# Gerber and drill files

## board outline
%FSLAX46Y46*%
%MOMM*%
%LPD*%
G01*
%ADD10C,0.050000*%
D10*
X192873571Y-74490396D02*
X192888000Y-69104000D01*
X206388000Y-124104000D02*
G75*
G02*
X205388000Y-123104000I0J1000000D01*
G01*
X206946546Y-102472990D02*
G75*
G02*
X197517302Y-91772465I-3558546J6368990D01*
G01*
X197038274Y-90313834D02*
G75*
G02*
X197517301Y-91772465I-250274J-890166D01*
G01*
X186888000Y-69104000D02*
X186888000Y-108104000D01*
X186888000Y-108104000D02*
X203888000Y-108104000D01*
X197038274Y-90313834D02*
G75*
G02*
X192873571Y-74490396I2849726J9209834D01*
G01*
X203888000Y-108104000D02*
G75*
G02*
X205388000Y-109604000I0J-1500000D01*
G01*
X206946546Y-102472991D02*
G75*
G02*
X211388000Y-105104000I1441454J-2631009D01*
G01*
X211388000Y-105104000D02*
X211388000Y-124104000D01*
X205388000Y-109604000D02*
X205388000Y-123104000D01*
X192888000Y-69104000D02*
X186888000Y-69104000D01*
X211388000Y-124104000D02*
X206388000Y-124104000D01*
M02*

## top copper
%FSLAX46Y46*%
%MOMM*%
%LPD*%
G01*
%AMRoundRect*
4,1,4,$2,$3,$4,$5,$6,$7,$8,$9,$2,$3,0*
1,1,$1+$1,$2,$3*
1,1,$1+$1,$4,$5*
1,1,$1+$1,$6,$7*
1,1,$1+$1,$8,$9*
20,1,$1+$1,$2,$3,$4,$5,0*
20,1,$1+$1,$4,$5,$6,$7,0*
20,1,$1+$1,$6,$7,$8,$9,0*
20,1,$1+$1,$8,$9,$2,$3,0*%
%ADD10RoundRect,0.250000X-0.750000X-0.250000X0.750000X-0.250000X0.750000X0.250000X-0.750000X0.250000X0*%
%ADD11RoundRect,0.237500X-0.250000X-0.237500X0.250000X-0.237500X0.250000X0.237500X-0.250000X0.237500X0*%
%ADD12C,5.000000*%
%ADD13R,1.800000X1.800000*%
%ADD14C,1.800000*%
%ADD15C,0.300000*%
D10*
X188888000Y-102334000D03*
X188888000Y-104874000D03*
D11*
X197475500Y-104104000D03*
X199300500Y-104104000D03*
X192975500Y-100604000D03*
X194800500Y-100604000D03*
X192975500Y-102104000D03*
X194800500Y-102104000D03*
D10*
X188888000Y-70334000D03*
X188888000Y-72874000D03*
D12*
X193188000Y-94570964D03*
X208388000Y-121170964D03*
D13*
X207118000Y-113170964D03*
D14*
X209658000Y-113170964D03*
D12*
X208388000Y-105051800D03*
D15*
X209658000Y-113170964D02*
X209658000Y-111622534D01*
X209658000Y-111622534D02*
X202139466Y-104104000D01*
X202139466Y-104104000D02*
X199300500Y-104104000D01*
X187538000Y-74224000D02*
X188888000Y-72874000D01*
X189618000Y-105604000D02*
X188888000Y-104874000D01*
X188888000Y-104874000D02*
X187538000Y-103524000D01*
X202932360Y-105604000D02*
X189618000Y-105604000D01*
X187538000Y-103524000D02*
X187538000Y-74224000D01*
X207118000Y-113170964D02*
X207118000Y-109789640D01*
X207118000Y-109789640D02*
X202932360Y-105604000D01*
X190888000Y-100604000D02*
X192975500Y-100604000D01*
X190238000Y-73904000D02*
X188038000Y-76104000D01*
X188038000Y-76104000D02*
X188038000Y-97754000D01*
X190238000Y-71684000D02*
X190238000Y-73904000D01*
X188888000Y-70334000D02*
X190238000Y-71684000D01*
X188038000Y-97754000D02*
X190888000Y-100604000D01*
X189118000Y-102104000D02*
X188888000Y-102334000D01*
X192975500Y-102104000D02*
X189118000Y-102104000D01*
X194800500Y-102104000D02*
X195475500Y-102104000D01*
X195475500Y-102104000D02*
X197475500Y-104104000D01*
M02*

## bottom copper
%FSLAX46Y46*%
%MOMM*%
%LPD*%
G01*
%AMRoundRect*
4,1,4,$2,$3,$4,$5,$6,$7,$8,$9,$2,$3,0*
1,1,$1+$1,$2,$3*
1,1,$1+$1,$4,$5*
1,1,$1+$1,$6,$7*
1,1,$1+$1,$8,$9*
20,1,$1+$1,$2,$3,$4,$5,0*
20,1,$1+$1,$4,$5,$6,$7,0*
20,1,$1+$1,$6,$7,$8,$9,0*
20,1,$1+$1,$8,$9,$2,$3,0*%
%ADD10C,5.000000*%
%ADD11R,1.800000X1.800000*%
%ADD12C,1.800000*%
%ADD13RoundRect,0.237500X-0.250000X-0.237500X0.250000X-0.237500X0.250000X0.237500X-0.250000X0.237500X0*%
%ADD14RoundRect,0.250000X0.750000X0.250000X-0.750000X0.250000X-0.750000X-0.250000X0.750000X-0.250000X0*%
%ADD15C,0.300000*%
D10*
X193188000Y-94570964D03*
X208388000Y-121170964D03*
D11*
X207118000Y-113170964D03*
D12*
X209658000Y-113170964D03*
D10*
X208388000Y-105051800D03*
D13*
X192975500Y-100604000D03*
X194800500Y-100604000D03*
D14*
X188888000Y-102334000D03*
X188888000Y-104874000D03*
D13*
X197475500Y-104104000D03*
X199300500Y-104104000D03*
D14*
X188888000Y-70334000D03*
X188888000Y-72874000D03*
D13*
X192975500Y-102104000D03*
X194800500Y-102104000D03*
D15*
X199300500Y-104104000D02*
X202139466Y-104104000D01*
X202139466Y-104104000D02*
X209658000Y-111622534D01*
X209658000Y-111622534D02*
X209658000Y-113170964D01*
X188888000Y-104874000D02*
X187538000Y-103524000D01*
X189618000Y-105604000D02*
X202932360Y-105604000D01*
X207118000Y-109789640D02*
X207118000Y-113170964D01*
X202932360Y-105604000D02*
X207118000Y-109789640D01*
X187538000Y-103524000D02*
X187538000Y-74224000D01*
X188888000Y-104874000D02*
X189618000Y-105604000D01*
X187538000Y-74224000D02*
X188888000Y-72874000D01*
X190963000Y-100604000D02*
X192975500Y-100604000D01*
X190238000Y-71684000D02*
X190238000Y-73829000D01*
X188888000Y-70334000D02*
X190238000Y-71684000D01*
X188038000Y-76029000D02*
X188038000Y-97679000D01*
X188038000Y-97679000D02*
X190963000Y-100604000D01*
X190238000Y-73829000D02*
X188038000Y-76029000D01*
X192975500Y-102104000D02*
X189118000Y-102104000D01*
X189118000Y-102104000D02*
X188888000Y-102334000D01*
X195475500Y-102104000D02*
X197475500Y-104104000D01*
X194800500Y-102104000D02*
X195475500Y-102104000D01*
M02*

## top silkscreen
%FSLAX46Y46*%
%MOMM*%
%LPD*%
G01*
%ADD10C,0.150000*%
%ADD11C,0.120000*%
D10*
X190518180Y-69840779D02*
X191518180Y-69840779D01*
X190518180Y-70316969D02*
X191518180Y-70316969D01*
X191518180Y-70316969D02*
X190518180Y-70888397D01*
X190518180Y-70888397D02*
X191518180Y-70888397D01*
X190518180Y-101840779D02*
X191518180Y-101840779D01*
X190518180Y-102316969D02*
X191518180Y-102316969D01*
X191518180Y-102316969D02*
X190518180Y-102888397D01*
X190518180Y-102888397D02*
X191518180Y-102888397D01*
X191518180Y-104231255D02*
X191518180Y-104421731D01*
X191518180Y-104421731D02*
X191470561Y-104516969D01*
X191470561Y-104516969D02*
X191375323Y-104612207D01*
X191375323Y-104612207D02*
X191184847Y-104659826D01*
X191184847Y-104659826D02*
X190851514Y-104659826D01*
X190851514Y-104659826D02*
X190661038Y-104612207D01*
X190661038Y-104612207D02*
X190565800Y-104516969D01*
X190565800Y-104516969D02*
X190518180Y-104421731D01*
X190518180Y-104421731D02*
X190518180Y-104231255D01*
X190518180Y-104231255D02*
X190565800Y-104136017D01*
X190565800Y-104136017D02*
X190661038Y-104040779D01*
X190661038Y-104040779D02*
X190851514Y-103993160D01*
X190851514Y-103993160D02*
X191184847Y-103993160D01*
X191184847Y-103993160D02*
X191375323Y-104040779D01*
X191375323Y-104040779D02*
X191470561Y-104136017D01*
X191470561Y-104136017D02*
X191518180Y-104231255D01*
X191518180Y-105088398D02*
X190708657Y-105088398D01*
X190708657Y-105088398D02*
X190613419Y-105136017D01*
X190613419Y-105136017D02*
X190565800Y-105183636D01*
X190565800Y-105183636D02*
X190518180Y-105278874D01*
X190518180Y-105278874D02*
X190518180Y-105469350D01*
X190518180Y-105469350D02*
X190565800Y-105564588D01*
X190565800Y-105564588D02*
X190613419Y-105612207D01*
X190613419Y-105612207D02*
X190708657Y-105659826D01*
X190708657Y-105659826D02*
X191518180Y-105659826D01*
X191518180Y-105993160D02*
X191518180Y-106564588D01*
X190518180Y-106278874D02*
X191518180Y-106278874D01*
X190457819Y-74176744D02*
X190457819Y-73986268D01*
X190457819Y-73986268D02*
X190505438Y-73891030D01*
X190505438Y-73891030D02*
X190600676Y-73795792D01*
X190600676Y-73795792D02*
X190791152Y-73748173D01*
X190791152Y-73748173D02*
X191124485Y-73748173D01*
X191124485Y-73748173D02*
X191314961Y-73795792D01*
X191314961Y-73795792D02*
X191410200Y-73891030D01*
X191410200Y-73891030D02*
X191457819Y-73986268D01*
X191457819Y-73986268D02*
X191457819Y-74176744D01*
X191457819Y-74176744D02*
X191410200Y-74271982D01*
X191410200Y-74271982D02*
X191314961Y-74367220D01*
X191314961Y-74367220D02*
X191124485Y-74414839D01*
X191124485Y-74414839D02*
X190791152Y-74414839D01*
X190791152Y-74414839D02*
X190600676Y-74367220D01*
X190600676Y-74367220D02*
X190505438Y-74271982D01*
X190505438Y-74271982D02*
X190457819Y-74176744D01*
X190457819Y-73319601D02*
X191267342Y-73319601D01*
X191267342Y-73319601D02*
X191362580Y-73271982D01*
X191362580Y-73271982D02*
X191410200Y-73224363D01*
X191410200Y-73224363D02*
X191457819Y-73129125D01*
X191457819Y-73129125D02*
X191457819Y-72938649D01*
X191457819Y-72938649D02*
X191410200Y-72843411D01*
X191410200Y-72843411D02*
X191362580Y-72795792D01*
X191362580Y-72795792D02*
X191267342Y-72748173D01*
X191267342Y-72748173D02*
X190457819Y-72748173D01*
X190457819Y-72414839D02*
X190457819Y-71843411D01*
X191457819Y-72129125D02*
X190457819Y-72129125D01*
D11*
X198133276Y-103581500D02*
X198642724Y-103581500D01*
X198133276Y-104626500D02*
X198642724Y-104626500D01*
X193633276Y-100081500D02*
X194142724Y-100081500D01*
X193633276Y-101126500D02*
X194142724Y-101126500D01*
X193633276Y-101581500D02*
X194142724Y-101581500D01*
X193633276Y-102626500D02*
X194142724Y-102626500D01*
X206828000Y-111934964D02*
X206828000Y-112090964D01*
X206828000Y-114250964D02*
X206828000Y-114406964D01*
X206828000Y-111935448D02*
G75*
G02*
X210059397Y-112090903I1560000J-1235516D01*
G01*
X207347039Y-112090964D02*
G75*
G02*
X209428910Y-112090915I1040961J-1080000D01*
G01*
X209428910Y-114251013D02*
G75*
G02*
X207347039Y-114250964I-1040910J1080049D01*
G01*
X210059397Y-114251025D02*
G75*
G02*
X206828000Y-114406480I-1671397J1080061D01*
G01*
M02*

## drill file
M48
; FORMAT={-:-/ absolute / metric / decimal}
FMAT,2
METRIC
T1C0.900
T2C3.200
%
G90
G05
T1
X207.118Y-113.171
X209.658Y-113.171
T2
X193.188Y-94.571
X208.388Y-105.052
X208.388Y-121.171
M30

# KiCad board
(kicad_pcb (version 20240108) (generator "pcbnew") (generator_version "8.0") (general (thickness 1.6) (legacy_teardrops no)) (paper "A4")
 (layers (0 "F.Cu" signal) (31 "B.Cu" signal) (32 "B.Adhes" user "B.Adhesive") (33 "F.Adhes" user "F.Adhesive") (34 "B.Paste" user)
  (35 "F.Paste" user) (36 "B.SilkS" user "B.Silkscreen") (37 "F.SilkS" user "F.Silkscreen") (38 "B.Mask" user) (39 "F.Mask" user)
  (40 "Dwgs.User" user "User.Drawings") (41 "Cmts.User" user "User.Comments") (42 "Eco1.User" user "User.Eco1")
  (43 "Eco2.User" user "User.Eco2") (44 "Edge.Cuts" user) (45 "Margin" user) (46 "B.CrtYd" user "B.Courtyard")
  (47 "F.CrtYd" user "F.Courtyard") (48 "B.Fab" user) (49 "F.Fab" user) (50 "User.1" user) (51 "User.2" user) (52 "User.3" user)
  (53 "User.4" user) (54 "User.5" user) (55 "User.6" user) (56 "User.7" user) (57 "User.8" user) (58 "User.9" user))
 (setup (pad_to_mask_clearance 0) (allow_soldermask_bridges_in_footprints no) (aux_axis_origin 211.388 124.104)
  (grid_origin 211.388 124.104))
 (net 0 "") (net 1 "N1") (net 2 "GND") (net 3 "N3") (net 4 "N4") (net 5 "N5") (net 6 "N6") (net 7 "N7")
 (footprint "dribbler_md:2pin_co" (layer "F.Cu") (at 188.888 103.604 -90)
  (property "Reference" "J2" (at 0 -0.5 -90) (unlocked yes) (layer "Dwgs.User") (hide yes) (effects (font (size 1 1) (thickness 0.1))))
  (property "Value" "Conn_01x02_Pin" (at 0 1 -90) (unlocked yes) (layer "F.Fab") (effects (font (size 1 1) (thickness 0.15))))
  (pad "1" smd roundrect (at -1.27 0) (size 2 1) (layers "F.Cu" "F.Paste" "F.Mask") (roundrect_rratio 0.25) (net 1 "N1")
   (thermal_bridge_angle 45))
  (pad "2" smd roundrect (at 1.27 0) (size 2 1) (layers "F.Cu" "F.Paste" "F.Mask") (roundrect_rratio 0.25) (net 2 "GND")
   (thermal_bridge_angle 45)))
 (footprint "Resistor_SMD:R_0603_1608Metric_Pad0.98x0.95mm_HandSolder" (layer "F.Cu") (at 198.388 104.104)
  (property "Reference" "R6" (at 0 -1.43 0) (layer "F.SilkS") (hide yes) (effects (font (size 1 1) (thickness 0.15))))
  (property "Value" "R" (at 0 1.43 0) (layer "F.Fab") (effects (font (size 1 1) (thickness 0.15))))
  (fp_line (start -0.254724 -0.5225) (end 0.254724 -0.5225) (stroke (width 0.12) (type solid)) (layer "F.SilkS"))
  (fp_line (start -0.254724 0.5225) (end 0.254724 0.5225) (stroke (width 0.12) (type solid)) (layer "F.SilkS"))
  (pad "1" smd roundrect (at -0.9125 0) (size 0.975 0.95) (layers "F.Cu" "F.Paste" "F.Mask") (roundrect_rratio 0.25) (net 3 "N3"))
  (pad "2" smd roundrect (at 0.9125 0) (size 0.975 0.95) (layers "F.Cu" "F.Paste" "F.Mask") (roundrect_rratio 0.25) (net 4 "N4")))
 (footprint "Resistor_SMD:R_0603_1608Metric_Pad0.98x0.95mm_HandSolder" (layer "F.Cu") (at 193.888 100.604)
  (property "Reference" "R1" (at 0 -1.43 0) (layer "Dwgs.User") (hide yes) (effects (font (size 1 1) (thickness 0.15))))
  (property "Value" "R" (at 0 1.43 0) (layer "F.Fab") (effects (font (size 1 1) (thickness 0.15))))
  (fp_line (start -0.254724 -0.5225) (end 0.254724 -0.5225) (stroke (width 0.12) (type solid)) (layer "F.SilkS"))
  (fp_line (start -0.254724 0.5225) (end 0.254724 0.5225) (stroke (width 0.12) (type solid)) (layer "F.SilkS"))
  (pad "1" smd roundrect (at -0.9125 0) (size 0.975 0.95) (layers "F.Cu" "F.Paste" "F.Mask") (roundrect_rratio 0.25) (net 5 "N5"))
  (pad "2" smd roundrect (at 0.9125 0) (size 0.975 0.95) (layers "F.Cu" "F.Paste" "F.Mask") (roundrect_rratio 0.25) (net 3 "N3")))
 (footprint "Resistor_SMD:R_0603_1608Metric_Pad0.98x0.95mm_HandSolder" (layer "F.Cu") (at 193.888 102.104)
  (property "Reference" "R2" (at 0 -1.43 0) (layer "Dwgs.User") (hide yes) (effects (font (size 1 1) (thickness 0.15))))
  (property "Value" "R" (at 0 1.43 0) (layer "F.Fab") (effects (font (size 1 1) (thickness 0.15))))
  (fp_line (start -0.254724 -0.5225) (end 0.254724 -0.5225) (stroke (width 0.12) (type solid)) (layer "F.SilkS"))
  (fp_line (start -0.254724 0.5225) (end 0.254724 0.5225) (stroke (width 0.12) (type solid)) (layer "F.SilkS"))
  (pad "1" smd roundrect (at -0.9125 0) (size 0.975 0.95) (layers "F.Cu" "F.Paste" "F.Mask") (roundrect_rratio 0.25) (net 1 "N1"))
  (pad "2" smd roundrect (at 0.9125 0) (size 0.975 0.95) (layers "F.Cu" "F.Paste" "F.Mask") (roundrect_rratio 0.25) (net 3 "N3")))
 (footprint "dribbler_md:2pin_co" (layer "F.Cu") (at 188.888 71.604 -90)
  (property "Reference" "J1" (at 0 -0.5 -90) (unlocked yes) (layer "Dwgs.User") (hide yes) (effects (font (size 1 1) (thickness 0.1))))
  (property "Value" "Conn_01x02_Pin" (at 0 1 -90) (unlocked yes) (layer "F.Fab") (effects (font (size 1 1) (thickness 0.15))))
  (pad "1" smd roundrect (at -1.27 0) (size 2 1) (layers "F.Cu" "F.Paste" "F.Mask") (roundrect_rratio 0.25) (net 5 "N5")
   (thermal_bridge_angle 45))
  (pad "2" smd roundrect (at 1.27 0) (size 2 1) (layers "F.Cu" "F.Paste" "F.Mask") (roundrect_rratio 0.25) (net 2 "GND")
   (thermal_bridge_angle 45)))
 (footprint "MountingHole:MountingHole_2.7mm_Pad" (layer "F.Cu") (at 193.188 94.570964)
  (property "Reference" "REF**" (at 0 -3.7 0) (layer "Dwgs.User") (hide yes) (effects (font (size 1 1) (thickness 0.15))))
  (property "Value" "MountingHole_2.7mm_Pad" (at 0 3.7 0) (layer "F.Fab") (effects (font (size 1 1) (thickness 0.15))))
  (pad "1" thru_hole circle (at 0 0) (size 5 5) (drill 3.2) (layers "*.Cu" "*.Mask") (remove_unused_layers no)))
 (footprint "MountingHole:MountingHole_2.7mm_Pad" (layer "F.Cu") (at 208.388 121.170964)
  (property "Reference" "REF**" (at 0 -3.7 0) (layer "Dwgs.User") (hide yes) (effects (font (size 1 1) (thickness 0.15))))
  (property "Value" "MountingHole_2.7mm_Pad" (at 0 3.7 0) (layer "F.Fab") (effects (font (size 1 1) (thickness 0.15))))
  (pad "1" thru_hole circle (at 0 0) (size 5 5) (drill 3.2) (layers "*.Cu" "*.Mask") (remove_unused_layers no)))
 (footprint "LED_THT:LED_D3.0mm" (layer "F.Cu") (at 207.118 113.170964)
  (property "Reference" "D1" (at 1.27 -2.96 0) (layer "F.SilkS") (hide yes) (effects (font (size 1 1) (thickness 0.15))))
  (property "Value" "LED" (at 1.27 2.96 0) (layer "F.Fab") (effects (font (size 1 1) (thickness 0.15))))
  (fp_line (start -0.29 -1.236) (end -0.29 -1.08) (stroke (width 0.12) (type solid)) (layer "F.SilkS"))
  (fp_line (start -0.29 1.08) (end -0.29 1.236) (stroke (width 0.12) (type solid)) (layer "F.SilkS"))
  (fp_arc (start -0.29 -1.235516) (mid 1.365624 -1.987701) (end 2.941397 -1.080061) (stroke (width 0.12) (type solid)) (layer "F.SilkS"))
  (fp_arc (start 0.229039 -1.08) (mid 1.269965 -1.5) (end 2.31091 -1.080049) (stroke (width 0.12) (type solid)) (layer "F.SilkS"))
  (fp_arc (start 2.31091 1.080049) (mid 1.269965 1.5) (end 0.229039 1.08) (stroke (width 0.12) (type solid)) (layer "F.SilkS"))
  (fp_arc (start 2.941397 1.080061) (mid 1.365624 1.987701) (end -0.29 1.235516) (stroke (width 0.12) (type solid)) (layer "F.SilkS"))
  (pad "1" thru_hole rect (at 0 0) (size 1.8 1.8) (drill 0.9) (layers "*.Cu" "*.Mask") (remove_unused_layers no) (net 2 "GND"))
  (pad "2" thru_hole circle (at 2.54 0) (size 1.8 1.8) (drill 0.9) (layers "*.Cu" "*.Mask") (remove_unused_layers no) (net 4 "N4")))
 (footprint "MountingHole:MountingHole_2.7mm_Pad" (layer "F.Cu") (at 208.388 105.0518)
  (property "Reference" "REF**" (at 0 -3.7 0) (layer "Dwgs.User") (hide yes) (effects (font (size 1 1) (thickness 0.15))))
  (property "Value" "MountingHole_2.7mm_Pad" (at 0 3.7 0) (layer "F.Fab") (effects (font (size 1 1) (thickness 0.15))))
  (pad "1" thru_hole circle (at 0 0) (size 5 5) (drill 3.2) (layers "*.Cu" "*.Mask") (remove_unused_layers no)))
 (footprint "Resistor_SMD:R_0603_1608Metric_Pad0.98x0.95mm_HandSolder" (layer "B.Cu") (at 193.888 100.604)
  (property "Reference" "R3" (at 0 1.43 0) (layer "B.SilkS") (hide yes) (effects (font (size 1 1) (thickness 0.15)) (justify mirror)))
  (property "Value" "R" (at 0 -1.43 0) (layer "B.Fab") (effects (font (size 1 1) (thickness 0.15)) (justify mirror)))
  (pad "1" smd roundrect (at -0.9125 0) (size 0.975 0.95) (layers "B.Cu" "B.Paste" "B.Mask") (roundrect_rratio 0.25) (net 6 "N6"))
  (pad "2" smd roundrect (at 0.9125 0) (size 0.975 0.95) (layers "B.Cu" "B.Paste" "B.Mask") (roundrect_rratio 0.25) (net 3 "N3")))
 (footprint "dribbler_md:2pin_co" (layer "B.Cu") (at 188.888 103.604 -90)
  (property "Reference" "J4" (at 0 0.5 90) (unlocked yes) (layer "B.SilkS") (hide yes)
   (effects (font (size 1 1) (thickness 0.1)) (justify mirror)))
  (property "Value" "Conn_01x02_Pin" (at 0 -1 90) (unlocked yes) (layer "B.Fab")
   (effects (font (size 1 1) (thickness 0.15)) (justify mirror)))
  (pad "1" smd roundrect (at -1.27 0 180) (size 2 1) (layers "B.Cu" "B.Paste" "B.Mask") (roundrect_rratio 0.25) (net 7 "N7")
   (thermal_bridge_angle 45))
  (pad "2" smd roundrect (at 1.27 0 180) (size 2 1) (layers "B.Cu" "B.Paste" "B.Mask") (roundrect_rratio 0.25) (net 2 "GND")
   (thermal_bridge_angle 45)))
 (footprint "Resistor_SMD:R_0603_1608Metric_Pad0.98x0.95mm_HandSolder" (layer "B.Cu") (at 198.388 104.104)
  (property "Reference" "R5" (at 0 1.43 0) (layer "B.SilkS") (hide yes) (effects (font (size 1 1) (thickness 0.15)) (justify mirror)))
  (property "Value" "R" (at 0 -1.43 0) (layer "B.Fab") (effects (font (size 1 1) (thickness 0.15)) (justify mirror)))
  (pad "1" smd roundrect (at -0.9125 0) (size 0.975 0.95) (layers "B.Cu" "B.Paste" "B.Mask") (roundrect_rratio 0.25) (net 3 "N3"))
  (pad "2" smd roundrect (at 0.9125 0) (size 0.975 0.95) (layers "B.Cu" "B.Paste" "B.Mask") (roundrect_rratio 0.25) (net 4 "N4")))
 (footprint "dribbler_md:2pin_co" (layer "B.Cu") (at 188.888 71.604 -90)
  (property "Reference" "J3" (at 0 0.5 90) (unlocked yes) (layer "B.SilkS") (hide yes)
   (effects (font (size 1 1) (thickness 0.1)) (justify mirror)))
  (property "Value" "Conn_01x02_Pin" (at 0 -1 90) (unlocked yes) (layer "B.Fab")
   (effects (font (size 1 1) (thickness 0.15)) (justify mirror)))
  (pad "1" smd roundrect (at -1.27 0 180) (size 2 1) (layers "B.Cu" "B.Paste" "B.Mask") (roundrect_rratio 0.25) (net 6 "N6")
   (thermal_bridge_angle 45))
  (pad "2" smd roundrect (at 1.27 0 180) (size 2 1) (layers "B.Cu" "B.Paste" "B.Mask") (roundrect_rratio 0.25) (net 2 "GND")
   (thermal_bridge_angle 45)))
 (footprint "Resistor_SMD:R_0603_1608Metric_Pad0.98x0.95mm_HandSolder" (layer "B.Cu") (at 193.888 102.104)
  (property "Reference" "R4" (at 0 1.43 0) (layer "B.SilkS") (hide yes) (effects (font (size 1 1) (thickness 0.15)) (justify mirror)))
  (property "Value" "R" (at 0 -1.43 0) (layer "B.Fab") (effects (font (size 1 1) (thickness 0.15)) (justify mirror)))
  (pad "1" smd roundrect (at -0.9125 0) (size 0.975 0.95) (layers "B.Cu" "B.Paste" "B.Mask") (roundrect_rratio 0.25) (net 7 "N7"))
  (pad "2" smd roundrect (at 0.9125 0) (size 0.975 0.95) (layers "B.Cu" "B.Paste" "B.Mask") (roundrect_rratio 0.25) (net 3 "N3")))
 (gr_line (start 192.873571 74.490396) (end 192.888 69.104) (stroke (width 0.05) (type default)) (layer "Edge.Cuts"))
 (gr_arc (start 206.388 124.104) (mid 205.680893 123.811107) (end 205.388 123.104) (stroke (width 0.05) (type default)) (layer "Edge.Cuts"))
 (gr_arc (start 206.946546 102.47299) (mid 197.914261 100.927429) (end 197.517302 91.772465) (stroke (width 0.05) (type default))
  (layer "Edge.Cuts"))
 (gr_arc (start 197.038274 90.313834) (mid 197.666517 90.915487) (end 197.517302 91.772465) (stroke (width 0.05) (type default))
  (layer "Edge.Cuts"))
 (gr_line (start 186.888 69.104) (end 186.888 108.104) (stroke (width 0.05) (type default)) (layer "Edge.Cuts"))
 (gr_line (start 186.888 108.104) (end 203.888 108.104) (stroke (width 0.05) (type default)) (layer "Edge.Cuts"))
 (gr_arc (start 197.038274 90.313834) (mid 190.564873 83.557832) (end 192.873571 74.490396) (stroke (width 0.05) (type default))
  (layer "Edge.Cuts"))
 (gr_arc (start 203.888 108.104) (mid 204.94866 108.54334) (end 205.388 109.604) (stroke (width 0.05) (type default)) (layer "Edge.Cuts"))
 (gr_arc (start 206.946546 102.472991) (mid 209.916993 102.52288) (end 211.388 105.104) (stroke (width 0.05) (type default))
  (layer "Edge.Cuts"))
 (gr_line (start 211.388 105.104) (end 211.388 124.104) (stroke (width 0.05) (type default)) (layer "Edge.Cuts"))
 (gr_line (start 205.388 109.604) (end 205.388 123.104) (stroke (width 0.05) (type default)) (layer "Edge.Cuts"))
 (gr_line (start 192.888 69.104) (end 186.888 69.104) (stroke (width 0.05) (type default)) (layer "Edge.Cuts"))
 (gr_line (start 211.388 124.104) (end 206.388 124.104) (stroke (width 0.05) (type default)) (layer "Edge.Cuts"))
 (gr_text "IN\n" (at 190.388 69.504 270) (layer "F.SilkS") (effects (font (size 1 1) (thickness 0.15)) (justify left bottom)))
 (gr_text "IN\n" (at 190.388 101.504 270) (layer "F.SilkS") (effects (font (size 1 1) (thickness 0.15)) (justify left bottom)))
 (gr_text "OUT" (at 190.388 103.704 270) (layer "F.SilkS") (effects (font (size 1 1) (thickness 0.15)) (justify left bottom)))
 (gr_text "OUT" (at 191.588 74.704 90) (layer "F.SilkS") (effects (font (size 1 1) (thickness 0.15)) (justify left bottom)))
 (segment (start 209.658 113.170964) (end 209.658 111.622534) (width 0.3) (layer "F.Cu") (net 4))
 (segment (start 209.658 111.622534) (end 202.139466 104.104) (width 0.3) (layer "F.Cu") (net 4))
 (segment (start 202.139466 104.104) (end 199.3005 104.104) (width 0.3) (layer "F.Cu") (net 4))
 (segment (start 199.3005 104.104) (end 202.139466 104.104) (width 0.3) (layer "B.Cu") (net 4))
 (segment (start 202.139466 104.104) (end 209.658 111.622534) (width 0.3) (layer "B.Cu") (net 4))
 (segment (start 209.658 111.622534) (end 209.658 113.170964) (width 0.3) (layer "B.Cu") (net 4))
 (segment (start 187.538 74.224) (end 188.888 72.874) (width 0.3) (layer "F.Cu") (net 2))
 (segment (start 189.618 105.604) (end 188.888 104.874) (width 0.3) (layer "F.Cu") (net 2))
 (segment (start 188.888 104.874) (end 187.538 103.524) (width 0.3) (layer "F.Cu") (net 2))
 (segment (start 202.93236 105.604) (end 189.618 105.604) (width 0.3) (layer "F.Cu") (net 2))
 (segment (start 187.538 103.524) (end 187.538 74.224) (width 0.3) (layer "F.Cu") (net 2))
 (segment (start 207.118 113.170964) (end 207.118 109.78964) (width 0.3) (layer "F.Cu") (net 2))
 (segment (start 207.118 109.78964) (end 202.93236 105.604) (width 0.3) (layer "F.Cu") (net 2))
 (segment (start 188.888 104.874) (end 187.538 103.524) (width 0.3) (layer "B.Cu") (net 2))
 (segment (start 189.618 105.604) (end 202.93236 105.604) (width 0.3) (layer "B.Cu") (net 2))
 (segment (start 207.118 109.78964) (end 207.118 113.170964) (width 0.3) (layer "B.Cu") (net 2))
 (segment (start 202.93236 105.604) (end 207.118 109.78964) (width 0.3) (layer "B.Cu") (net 2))
 (segment (start 187.538 103.524) (end 187.538 74.224) (width 0.3) (layer "B.Cu") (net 2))
 (segment (start 188.888 104.874) (end 189.618 105.604) (width 0.3) (layer "B.Cu") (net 2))
 (segment (start 187.538 74.224) (end 188.888 72.874) (width 0.3) (layer "B.Cu") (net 2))
 (segment (start 190.888 100.604) (end 192.9755 100.604) (width 0.3) (layer "F.Cu") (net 5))
 (segment (start 190.238 73.904) (end 188.038 76.104) (width 0.3) (layer "F.Cu") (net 5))
 (segment (start 188.038 76.104) (end 188.038 97.754) (width 0.3) (layer "F.Cu") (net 5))
 (segment (start 190.238 71.684) (end 190.238 73.904) (width 0.3) (layer "F.Cu") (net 5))
 (segment (start 188.888 70.334) (end 190.238 71.684) (width 0.3) (layer "F.Cu") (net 5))
 (segment (start 188.038 97.754) (end 190.888 100.604) (width 0.3) (layer "F.Cu") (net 5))
 (segment (start 189.118 102.104) (end 188.888 102.334) (width 0.3) (layer "F.Cu") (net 1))
 (segment (start 192.9755 102.104) (end 189.118 102.104) (width 0.3) (layer "F.Cu") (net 1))
 (segment (start 190.963 100.604) (end 192.9755 100.604) (width 0.3) (layer "B.Cu") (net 6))
 (segment (start 190.238 71.684) (end 190.238 73.829) (width 0.3) (layer "B.Cu") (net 6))
 (segment (start 188.888 70.334) (end 190.238 71.684) (width 0.3) (layer "B.Cu") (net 6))
 (segment (start 188.038 76.029) (end 188.038 97.679) (width 0.3) (layer "B.Cu") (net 6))
 (segment (start 188.038 97.679) (end 190.963 100.604) (width 0.3) (layer "B.Cu") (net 6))
 (segment (start 190.238 73.829) (end 188.038 76.029) (width 0.3) (layer "B.Cu") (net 6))
 (segment (start 192.9755 102.104) (end 189.118 102.104) (width 0.3) (layer "B.Cu") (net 7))
 (segment (start 189.118 102.104) (end 188.888 102.334) (width 0.3) (layer "B.Cu") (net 7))
 (segment (start 194.8005 102.104) (end 195.4755 102.104) (width 0.3) (layer "F.Cu") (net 3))
 (segment (start 195.4755 102.104) (end 197.4755 104.104) (width 0.3) (layer "F.Cu") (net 3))
 (segment (start 195.4755 102.104) (end 197.4755 104.104) (width 0.3) (layer "B.Cu") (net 3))
 (segment (start 194.8005 102.104) (end 195.4755 102.104) (width 0.3) (layer "B.Cu") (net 3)))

